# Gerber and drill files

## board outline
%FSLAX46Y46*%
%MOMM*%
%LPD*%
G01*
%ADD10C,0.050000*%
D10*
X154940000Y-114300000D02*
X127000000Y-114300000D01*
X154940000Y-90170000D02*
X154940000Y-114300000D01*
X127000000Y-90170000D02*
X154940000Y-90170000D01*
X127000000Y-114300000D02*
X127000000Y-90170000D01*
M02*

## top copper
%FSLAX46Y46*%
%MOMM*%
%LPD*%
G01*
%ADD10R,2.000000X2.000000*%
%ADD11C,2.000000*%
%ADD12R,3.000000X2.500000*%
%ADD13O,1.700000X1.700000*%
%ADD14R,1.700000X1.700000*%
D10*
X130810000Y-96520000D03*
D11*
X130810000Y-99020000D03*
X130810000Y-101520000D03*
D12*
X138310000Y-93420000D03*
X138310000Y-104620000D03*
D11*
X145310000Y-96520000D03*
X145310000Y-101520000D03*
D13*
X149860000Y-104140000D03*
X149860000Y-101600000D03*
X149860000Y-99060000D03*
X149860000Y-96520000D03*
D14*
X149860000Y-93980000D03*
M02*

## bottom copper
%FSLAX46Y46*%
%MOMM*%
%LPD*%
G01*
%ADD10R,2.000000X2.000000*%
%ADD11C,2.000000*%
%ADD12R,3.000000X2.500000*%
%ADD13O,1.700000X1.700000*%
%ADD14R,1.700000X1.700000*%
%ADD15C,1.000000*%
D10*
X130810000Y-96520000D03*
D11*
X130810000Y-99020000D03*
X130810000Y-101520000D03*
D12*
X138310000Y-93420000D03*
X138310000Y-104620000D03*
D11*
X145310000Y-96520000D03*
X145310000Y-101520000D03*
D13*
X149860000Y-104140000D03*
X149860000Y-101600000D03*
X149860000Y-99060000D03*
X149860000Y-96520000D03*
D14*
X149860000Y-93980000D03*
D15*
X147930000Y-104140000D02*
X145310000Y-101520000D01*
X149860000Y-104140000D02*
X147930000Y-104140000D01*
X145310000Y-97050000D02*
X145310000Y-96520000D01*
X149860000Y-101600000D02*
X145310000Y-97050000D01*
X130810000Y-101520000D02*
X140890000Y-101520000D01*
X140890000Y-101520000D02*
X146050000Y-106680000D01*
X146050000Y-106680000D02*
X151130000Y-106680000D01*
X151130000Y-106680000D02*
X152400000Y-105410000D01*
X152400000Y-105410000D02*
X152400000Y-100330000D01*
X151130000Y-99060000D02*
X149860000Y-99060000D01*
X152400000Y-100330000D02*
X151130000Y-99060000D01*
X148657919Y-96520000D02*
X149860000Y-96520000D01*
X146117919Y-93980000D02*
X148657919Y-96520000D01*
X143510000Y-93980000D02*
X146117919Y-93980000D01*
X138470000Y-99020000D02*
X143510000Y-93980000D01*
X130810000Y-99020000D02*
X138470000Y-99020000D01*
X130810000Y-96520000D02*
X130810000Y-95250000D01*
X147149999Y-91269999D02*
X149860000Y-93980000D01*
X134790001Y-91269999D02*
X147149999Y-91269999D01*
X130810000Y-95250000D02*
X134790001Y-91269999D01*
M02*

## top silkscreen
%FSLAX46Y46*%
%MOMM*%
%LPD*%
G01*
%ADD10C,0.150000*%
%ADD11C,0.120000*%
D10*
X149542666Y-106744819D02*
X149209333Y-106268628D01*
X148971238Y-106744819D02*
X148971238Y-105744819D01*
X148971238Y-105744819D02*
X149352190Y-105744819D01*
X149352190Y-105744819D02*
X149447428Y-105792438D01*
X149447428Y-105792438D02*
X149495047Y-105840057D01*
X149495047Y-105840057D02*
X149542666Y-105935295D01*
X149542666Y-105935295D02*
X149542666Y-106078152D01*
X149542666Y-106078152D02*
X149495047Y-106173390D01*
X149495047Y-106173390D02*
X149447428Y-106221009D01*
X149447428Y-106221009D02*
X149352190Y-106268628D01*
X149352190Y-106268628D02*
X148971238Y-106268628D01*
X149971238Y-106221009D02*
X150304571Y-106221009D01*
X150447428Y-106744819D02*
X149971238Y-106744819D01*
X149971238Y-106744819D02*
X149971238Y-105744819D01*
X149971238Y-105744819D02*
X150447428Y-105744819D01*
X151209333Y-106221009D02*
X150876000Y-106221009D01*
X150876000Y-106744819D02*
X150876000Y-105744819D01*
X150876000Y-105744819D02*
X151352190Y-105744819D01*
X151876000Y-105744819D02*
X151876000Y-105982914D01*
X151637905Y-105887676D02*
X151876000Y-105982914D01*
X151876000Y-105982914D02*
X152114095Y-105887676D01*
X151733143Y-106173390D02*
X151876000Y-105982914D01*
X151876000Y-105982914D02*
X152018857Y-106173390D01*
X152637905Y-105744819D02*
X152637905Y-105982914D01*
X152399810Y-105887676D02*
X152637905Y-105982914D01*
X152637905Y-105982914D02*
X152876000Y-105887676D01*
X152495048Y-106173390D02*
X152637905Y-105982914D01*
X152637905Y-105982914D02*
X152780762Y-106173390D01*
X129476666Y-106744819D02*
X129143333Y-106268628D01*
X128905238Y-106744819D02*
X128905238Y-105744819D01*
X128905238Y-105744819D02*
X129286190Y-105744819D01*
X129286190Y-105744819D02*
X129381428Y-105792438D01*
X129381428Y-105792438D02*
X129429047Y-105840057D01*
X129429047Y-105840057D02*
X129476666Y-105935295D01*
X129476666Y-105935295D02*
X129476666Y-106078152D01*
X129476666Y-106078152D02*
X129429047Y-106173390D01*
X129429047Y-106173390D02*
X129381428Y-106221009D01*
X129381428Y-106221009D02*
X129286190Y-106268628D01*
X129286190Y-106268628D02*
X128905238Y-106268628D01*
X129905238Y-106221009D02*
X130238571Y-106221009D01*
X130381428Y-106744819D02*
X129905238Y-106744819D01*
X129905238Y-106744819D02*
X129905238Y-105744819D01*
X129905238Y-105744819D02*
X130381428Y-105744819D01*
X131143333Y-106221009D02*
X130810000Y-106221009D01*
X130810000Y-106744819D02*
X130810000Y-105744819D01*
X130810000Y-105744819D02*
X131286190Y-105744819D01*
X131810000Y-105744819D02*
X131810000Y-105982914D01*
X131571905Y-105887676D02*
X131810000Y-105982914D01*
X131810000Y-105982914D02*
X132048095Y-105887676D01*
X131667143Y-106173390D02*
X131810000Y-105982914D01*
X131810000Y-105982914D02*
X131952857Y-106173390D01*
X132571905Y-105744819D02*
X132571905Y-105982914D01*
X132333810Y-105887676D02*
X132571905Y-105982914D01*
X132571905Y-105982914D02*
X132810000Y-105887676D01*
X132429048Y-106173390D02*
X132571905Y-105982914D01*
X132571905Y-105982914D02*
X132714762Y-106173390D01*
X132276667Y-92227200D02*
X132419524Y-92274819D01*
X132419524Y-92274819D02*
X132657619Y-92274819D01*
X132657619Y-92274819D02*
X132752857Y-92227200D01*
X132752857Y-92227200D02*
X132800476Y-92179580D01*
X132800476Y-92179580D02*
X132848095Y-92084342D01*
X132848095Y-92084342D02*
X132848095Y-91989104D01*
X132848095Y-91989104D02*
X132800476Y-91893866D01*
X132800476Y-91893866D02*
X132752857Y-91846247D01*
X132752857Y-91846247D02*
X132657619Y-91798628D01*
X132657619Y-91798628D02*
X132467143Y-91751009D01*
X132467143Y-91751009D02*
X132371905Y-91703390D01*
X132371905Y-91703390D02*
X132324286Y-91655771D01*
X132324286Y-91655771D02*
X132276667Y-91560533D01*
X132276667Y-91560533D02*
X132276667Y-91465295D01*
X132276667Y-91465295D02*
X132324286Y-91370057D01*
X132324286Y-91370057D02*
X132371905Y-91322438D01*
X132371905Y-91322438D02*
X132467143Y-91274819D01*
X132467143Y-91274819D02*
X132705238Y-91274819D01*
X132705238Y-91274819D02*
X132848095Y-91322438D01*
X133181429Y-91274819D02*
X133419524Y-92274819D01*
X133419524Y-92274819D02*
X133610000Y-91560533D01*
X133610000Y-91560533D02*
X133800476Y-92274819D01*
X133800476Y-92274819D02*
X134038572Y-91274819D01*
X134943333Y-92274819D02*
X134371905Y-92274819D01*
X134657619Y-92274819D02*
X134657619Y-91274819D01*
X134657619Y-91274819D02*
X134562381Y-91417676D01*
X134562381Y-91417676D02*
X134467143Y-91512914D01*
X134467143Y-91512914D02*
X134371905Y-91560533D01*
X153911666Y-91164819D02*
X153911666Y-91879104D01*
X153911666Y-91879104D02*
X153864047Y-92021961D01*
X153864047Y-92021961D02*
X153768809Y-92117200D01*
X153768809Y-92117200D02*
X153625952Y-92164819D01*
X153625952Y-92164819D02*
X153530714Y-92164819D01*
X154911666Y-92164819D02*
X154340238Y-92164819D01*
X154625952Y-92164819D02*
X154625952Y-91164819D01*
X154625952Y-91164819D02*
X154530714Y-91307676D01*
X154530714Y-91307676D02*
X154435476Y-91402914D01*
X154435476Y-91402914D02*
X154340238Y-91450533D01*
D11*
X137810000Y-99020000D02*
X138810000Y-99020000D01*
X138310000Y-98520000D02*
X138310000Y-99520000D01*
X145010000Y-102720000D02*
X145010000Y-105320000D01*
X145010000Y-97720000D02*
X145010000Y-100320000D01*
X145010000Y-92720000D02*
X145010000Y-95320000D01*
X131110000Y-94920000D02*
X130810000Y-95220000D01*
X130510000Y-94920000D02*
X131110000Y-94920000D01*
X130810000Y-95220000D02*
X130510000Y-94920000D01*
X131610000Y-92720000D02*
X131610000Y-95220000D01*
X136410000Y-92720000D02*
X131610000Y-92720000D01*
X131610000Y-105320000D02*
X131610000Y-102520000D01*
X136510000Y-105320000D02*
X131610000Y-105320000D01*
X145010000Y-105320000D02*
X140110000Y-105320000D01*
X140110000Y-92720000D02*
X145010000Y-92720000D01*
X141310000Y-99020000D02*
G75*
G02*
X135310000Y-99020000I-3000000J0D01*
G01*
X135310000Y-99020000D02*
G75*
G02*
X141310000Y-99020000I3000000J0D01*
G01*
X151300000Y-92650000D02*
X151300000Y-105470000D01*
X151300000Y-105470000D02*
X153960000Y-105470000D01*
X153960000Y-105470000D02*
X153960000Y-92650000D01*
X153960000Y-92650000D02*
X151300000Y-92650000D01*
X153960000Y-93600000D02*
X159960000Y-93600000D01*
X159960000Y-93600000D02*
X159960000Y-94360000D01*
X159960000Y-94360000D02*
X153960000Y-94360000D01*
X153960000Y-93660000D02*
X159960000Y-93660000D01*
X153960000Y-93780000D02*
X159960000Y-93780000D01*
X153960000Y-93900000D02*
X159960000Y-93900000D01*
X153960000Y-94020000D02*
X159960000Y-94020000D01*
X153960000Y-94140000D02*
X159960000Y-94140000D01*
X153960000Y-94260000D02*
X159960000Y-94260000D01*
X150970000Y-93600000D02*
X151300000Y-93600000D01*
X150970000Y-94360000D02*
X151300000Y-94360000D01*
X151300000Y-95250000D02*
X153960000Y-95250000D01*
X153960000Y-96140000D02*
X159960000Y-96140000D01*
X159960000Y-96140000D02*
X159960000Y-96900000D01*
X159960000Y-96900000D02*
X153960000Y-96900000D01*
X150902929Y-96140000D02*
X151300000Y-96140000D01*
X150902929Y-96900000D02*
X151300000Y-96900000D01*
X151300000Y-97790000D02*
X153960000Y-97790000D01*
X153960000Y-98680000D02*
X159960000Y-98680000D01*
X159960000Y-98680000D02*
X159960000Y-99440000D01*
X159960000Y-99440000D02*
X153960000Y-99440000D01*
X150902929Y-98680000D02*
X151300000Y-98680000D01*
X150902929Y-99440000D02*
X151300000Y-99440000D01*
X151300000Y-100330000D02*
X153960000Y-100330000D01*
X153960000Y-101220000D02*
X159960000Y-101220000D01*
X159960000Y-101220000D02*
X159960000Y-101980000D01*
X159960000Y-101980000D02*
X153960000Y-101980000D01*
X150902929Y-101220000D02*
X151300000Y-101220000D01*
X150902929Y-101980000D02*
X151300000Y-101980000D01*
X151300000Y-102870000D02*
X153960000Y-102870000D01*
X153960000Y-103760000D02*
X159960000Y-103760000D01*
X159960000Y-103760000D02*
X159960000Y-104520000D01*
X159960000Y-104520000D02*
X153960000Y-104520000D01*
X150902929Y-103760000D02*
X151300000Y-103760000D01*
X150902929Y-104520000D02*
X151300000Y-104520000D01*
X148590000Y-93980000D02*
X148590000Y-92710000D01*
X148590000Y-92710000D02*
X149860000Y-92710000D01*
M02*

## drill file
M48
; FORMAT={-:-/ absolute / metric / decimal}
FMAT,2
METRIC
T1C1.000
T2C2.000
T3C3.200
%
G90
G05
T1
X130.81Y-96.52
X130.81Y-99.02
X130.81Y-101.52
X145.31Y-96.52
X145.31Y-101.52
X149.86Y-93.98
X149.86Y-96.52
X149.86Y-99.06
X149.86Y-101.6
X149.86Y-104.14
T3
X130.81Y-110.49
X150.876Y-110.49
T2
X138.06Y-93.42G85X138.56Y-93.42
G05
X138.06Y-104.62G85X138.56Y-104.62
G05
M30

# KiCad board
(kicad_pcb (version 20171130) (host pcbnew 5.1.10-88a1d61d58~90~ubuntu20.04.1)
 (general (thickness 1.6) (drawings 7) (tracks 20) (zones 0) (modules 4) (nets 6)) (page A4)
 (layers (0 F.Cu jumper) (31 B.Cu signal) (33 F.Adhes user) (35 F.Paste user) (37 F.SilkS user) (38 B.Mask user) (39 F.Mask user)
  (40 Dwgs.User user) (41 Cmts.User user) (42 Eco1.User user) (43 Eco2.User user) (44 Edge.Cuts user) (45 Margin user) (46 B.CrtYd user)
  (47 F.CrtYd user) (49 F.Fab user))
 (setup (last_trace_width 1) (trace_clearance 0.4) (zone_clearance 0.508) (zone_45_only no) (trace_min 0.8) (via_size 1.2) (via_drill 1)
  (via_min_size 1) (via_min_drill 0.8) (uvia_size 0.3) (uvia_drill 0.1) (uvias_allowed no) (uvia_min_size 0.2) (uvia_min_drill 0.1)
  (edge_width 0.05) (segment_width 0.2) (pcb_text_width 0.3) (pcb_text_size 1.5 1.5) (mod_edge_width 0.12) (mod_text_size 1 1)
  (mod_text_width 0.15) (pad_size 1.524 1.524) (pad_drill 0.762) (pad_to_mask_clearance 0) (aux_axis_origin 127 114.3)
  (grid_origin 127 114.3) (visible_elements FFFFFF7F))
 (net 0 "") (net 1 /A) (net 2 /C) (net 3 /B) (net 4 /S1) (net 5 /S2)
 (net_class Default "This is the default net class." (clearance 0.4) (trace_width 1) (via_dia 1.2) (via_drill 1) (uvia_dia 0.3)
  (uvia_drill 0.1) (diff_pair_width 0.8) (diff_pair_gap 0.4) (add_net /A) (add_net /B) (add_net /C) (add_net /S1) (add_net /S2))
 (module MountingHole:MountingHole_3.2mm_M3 (layer F.Cu) (at 150.876 110.49)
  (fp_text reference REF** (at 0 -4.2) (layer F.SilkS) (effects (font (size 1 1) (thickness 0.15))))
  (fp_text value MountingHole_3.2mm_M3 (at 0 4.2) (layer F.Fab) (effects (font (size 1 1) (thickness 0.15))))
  (pad 1 np_thru_hole circle (at 0 0) (size 3.2 3.2) (drill 3.2) (layers *.Cu *.Mask)))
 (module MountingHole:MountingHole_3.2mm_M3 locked (layer F.Cu) (at 130.81 110.49)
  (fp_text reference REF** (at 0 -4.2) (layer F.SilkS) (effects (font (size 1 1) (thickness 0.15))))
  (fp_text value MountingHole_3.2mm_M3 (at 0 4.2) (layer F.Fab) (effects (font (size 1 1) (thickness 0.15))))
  (pad 1 np_thru_hole circle (at 0 0) (size 3.2 3.2) (drill 3.2) (layers *.Cu *.Mask)))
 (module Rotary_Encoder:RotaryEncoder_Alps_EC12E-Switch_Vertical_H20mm (layer F.Cu) (at 130.81 96.52)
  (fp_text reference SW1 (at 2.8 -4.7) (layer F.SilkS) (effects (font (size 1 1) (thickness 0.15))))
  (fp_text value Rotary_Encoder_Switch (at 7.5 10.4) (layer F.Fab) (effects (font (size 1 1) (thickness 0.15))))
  (fp_line (start 7 2.5) (end 8 2.5) (layer F.SilkS) (width 0.12))
  (fp_line (start 7.5 2) (end 7.5 3) (layer F.SilkS) (width 0.12))
  (fp_line (start 14.2 6.2) (end 14.2 8.8) (layer F.SilkS) (width 0.12))
  (fp_line (start 14.2 1.2) (end 14.2 3.8) (layer F.SilkS) (width 0.12))
  (fp_line (start 14.2 -3.8) (end 14.2 -1.2) (layer F.SilkS) (width 0.12))
  (fp_line (start 0.3 -1.6) (end 0 -1.3) (layer F.SilkS) (width 0.12))
  (fp_line (start -0.3 -1.6) (end 0.3 -1.6) (layer F.SilkS) (width 0.12))
  (fp_line (start 0 -1.3) (end -0.3 -1.6) (layer F.SilkS) (width 0.12))
  (fp_line (start 0.8 -3.8) (end 0.8 -1.3) (layer F.SilkS) (width 0.12))
  (fp_line (start 5.6 -3.8) (end 0.8 -3.8) (layer F.SilkS) (width 0.12))
  (fp_line (start 0.8 8.8) (end 0.8 6) (layer F.SilkS) (width 0.12))
  (fp_line (start 5.7 8.8) (end 0.8 8.8) (layer F.SilkS) (width 0.12))
  (fp_line (start 14.2 8.8) (end 9.3 8.8) (layer F.SilkS) (width 0.12))
  (fp_line (start 9.3 -3.8) (end 14.2 -3.8) (layer F.SilkS) (width 0.12))
  (fp_circle (center 7.5 2.5) (end 10.5 2.5) (layer F.SilkS) (width 0.12))
  (pad A thru_hole rect (at 0 0) (size 2 2) (drill 1) (layers *.Cu *.Mask) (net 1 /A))
  (pad C thru_hole circle (at 0 2.5) (size 2 2) (drill 1) (layers *.Cu *.Mask) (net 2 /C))
  (pad B thru_hole circle (at 0 5) (size 2 2) (drill 1) (layers *.Cu *.Mask) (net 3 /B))
  (pad MP thru_hole rect (at 7.5 -3.1) (size 3 2.5) (drill oval 2.5 2) (layers *.Cu *.Mask))
  (pad MP thru_hole rect (at 7.5 8.1) (size 3 2.5) (drill oval 2.5 2) (layers *.Cu *.Mask))
  (pad S1 thru_hole circle (at 14.5 0) (size 2 2) (drill 1) (layers *.Cu *.Mask) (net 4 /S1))
  (pad S2 thru_hole circle (at 14.5 5) (size 2 2) (drill 1) (layers *.Cu *.Mask) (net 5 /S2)))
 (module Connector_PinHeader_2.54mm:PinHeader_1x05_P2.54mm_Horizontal (layer F.Cu) (at 149.86 93.98)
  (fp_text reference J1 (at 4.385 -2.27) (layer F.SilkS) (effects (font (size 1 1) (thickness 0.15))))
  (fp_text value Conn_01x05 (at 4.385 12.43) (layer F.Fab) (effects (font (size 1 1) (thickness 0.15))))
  (fp_line (start 1.44 -1.33) (end 1.44 11.49) (layer F.SilkS) (width 0.12))
  (fp_line (start 1.44 11.49) (end 4.1 11.49) (layer F.SilkS) (width 0.12))
  (fp_line (start 4.1 11.49) (end 4.1 -1.33) (layer F.SilkS) (width 0.12))
  (fp_line (start 4.1 -1.33) (end 1.44 -1.33) (layer F.SilkS) (width 0.12))
  (fp_line (start 4.1 -0.38) (end 10.1 -0.38) (layer F.SilkS) (width 0.12))
  (fp_line (start 10.1 -0.38) (end 10.1 0.38) (layer F.SilkS) (width 0.12))
  (fp_line (start 10.1 0.38) (end 4.1 0.38) (layer F.SilkS) (width 0.12))
  (fp_line (start 4.1 -0.32) (end 10.1 -0.32) (layer F.SilkS) (width 0.12))
  (fp_line (start 4.1 -0.2) (end 10.1 -0.2) (layer F.SilkS) (width 0.12))
  (fp_line (start 4.1 -0.08) (end 10.1 -0.08) (layer F.SilkS) (width 0.12))
  (fp_line (start 4.1 0.04) (end 10.1 0.04) (layer F.SilkS) (width 0.12))
  (fp_line (start 4.1 0.16) (end 10.1 0.16) (layer F.SilkS) (width 0.12))
  (fp_line (start 4.1 0.28) (end 10.1 0.28) (layer F.SilkS) (width 0.12))
  (fp_line (start 1.11 -0.38) (end 1.44 -0.38) (layer F.SilkS) (width 0.12))
  (fp_line (start 1.11 0.38) (end 1.44 0.38) (layer F.SilkS) (width 0.12))
  (fp_line (start 1.44 1.27) (end 4.1 1.27) (layer F.SilkS) (width 0.12))
  (fp_line (start 4.1 2.16) (end 10.1 2.16) (layer F.SilkS) (width 0.12))
  (fp_line (start 10.1 2.16) (end 10.1 2.92) (layer F.SilkS) (width 0.12))
  (fp_line (start 10.1 2.92) (end 4.1 2.92) (layer F.SilkS) (width 0.12))
  (fp_line (start 1.042929 2.16) (end 1.44 2.16) (layer F.SilkS) (width 0.12))
  (fp_line (start 1.042929 2.92) (end 1.44 2.92) (layer F.SilkS) (width 0.12))
  (fp_line (start 1.44 3.81) (end 4.1 3.81) (layer F.SilkS) (width 0.12))
  (fp_line (start 4.1 4.7) (end 10.1 4.7) (layer F.SilkS) (width 0.12))
  (fp_line (start 10.1 4.7) (end 10.1 5.46) (layer F.SilkS) (width 0.12))
  (fp_line (start 10.1 5.46) (end 4.1 5.46) (layer F.SilkS) (width 0.12))
  (fp_line (start 1.042929 4.7) (end 1.44 4.7) (layer F.SilkS) (width 0.12))
  (fp_line (start 1.042929 5.46) (end 1.44 5.46) (layer F.SilkS) (width 0.12))
  (fp_line (start 1.44 6.35) (end 4.1 6.35) (layer F.SilkS) (width 0.12))
  (fp_line (start 4.1 7.24) (end 10.1 7.24) (layer F.SilkS) (width 0.12))
  (fp_line (start 10.1 7.24) (end 10.1 8) (layer F.SilkS) (width 0.12))
  (fp_line (start 10.1 8) (end 4.1 8) (layer F.SilkS) (width 0.12))
  (fp_line (start 1.042929 7.24) (end 1.44 7.24) (layer F.SilkS) (width 0.12))
  (fp_line (start 1.042929 8) (end 1.44 8) (layer F.SilkS) (width 0.12))
  (fp_line (start 1.44 8.89) (end 4.1 8.89) (layer F.SilkS) (width 0.12))
  (fp_line (start 4.1 9.78) (end 10.1 9.78) (layer F.SilkS) (width 0.12))
  (fp_line (start 10.1 9.78) (end 10.1 10.54) (layer F.SilkS) (width 0.12))
  (fp_line (start 10.1 10.54) (end 4.1 10.54) (layer F.SilkS) (width 0.12))
  (fp_line (start 1.042929 9.78) (end 1.44 9.78) (layer F.SilkS) (width 0.12))
  (fp_line (start 1.042929 10.54) (end 1.44 10.54) (layer F.SilkS) (width 0.12))
  (fp_line (start -1.27 0) (end -1.27 -1.27) (layer F.SilkS) (width 0.12))
  (fp_line (start -1.27 -1.27) (end 0 -1.27) (layer F.SilkS) (width 0.12))
  (pad 5 thru_hole oval (at 0 10.16) (size 1.7 1.7) (drill 1) (layers *.Cu *.Mask) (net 5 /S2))
  (pad 4 thru_hole oval (at 0 7.62) (size 1.7 1.7) (drill 1) (layers *.Cu *.Mask) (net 4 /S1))
  (pad 3 thru_hole oval (at 0 5.08) (size 1.7 1.7) (drill 1) (layers *.Cu *.Mask) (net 3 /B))
  (pad 2 thru_hole oval (at 0 2.54) (size 1.7 1.7) (drill 1) (layers *.Cu *.Mask) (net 2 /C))
  (pad 1 thru_hole rect (at 0 0) (size 1.7 1.7) (drill 1) (layers *.Cu *.Mask) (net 1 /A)))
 (gr_line (start 154.94 114.3) (end 127 114.3) (layer Edge.Cuts) (width 0.05))
 (gr_line (start 154.94 90.17) (end 154.94 114.3) (layer Edge.Cuts) (width 0.05))
 (gr_line (start 127 90.17) (end 154.94 90.17) (layer Edge.Cuts) (width 0.05))
 (gr_line (start 127 114.3) (end 127 90.17) (layer Edge.Cuts) (width 0.05))
 (segment (start 147.93 104.14) (end 145.31 101.52) (width 1) (layer B.Cu) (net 5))
 (segment (start 149.86 104.14) (end 147.93 104.14) (width 1) (layer B.Cu) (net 5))
 (segment (start 145.31 97.05) (end 145.31 96.52) (width 1) (layer B.Cu) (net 4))
 (segment (start 149.86 101.6) (end 145.31 97.05) (width 1) (layer B.Cu) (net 4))
 (segment (start 130.81 101.52) (end 140.89 101.52) (width 1) (layer B.Cu) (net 3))
 (segment (start 140.89 101.52) (end 146.05 106.68) (width 1) (layer B.Cu) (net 3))
 (segment (start 146.05 106.68) (end 151.13 106.68) (width 1) (layer B.Cu) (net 3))
 (segment (start 151.13 106.68) (end 152.4 105.41) (width 1) (layer B.Cu) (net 3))
 (segment (start 152.4 105.41) (end 152.4 100.33) (width 1) (layer B.Cu) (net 3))
 (segment (start 151.13 99.06) (end 149.86 99.06) (width 1) (layer B.Cu) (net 3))
 (segment (start 152.4 100.33) (end 151.13 99.06) (width 1) (layer B.Cu) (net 3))
 (segment (start 148.657919 96.52) (end 149.86 96.52) (width 1) (layer B.Cu) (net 2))
 (segment (start 146.117919 93.98) (end 148.657919 96.52) (width 1) (layer B.Cu) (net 2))
 (segment (start 143.51 93.98) (end 146.117919 93.98) (width 1) (layer B.Cu) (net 2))
 (segment (start 138.47 99.02) (end 143.51 93.98) (width 1) (layer B.Cu) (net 2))
 (segment (start 130.81 99.02) (end 138.47 99.02) (width 1) (layer B.Cu) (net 2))
 (segment (start 130.81 96.52) (end 130.81 95.25) (width 1) (layer B.Cu) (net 1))
 (segment (start 147.149999 91.269999) (end 149.86 93.98) (width 1) (layer B.Cu) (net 1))
 (segment (start 134.790001 91.269999) (end 147.149999 91.269999) (width 1) (layer B.Cu) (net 1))
 (segment (start 130.81 95.25) (end 134.790001 91.269999) (width 1) (layer B.Cu) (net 1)))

